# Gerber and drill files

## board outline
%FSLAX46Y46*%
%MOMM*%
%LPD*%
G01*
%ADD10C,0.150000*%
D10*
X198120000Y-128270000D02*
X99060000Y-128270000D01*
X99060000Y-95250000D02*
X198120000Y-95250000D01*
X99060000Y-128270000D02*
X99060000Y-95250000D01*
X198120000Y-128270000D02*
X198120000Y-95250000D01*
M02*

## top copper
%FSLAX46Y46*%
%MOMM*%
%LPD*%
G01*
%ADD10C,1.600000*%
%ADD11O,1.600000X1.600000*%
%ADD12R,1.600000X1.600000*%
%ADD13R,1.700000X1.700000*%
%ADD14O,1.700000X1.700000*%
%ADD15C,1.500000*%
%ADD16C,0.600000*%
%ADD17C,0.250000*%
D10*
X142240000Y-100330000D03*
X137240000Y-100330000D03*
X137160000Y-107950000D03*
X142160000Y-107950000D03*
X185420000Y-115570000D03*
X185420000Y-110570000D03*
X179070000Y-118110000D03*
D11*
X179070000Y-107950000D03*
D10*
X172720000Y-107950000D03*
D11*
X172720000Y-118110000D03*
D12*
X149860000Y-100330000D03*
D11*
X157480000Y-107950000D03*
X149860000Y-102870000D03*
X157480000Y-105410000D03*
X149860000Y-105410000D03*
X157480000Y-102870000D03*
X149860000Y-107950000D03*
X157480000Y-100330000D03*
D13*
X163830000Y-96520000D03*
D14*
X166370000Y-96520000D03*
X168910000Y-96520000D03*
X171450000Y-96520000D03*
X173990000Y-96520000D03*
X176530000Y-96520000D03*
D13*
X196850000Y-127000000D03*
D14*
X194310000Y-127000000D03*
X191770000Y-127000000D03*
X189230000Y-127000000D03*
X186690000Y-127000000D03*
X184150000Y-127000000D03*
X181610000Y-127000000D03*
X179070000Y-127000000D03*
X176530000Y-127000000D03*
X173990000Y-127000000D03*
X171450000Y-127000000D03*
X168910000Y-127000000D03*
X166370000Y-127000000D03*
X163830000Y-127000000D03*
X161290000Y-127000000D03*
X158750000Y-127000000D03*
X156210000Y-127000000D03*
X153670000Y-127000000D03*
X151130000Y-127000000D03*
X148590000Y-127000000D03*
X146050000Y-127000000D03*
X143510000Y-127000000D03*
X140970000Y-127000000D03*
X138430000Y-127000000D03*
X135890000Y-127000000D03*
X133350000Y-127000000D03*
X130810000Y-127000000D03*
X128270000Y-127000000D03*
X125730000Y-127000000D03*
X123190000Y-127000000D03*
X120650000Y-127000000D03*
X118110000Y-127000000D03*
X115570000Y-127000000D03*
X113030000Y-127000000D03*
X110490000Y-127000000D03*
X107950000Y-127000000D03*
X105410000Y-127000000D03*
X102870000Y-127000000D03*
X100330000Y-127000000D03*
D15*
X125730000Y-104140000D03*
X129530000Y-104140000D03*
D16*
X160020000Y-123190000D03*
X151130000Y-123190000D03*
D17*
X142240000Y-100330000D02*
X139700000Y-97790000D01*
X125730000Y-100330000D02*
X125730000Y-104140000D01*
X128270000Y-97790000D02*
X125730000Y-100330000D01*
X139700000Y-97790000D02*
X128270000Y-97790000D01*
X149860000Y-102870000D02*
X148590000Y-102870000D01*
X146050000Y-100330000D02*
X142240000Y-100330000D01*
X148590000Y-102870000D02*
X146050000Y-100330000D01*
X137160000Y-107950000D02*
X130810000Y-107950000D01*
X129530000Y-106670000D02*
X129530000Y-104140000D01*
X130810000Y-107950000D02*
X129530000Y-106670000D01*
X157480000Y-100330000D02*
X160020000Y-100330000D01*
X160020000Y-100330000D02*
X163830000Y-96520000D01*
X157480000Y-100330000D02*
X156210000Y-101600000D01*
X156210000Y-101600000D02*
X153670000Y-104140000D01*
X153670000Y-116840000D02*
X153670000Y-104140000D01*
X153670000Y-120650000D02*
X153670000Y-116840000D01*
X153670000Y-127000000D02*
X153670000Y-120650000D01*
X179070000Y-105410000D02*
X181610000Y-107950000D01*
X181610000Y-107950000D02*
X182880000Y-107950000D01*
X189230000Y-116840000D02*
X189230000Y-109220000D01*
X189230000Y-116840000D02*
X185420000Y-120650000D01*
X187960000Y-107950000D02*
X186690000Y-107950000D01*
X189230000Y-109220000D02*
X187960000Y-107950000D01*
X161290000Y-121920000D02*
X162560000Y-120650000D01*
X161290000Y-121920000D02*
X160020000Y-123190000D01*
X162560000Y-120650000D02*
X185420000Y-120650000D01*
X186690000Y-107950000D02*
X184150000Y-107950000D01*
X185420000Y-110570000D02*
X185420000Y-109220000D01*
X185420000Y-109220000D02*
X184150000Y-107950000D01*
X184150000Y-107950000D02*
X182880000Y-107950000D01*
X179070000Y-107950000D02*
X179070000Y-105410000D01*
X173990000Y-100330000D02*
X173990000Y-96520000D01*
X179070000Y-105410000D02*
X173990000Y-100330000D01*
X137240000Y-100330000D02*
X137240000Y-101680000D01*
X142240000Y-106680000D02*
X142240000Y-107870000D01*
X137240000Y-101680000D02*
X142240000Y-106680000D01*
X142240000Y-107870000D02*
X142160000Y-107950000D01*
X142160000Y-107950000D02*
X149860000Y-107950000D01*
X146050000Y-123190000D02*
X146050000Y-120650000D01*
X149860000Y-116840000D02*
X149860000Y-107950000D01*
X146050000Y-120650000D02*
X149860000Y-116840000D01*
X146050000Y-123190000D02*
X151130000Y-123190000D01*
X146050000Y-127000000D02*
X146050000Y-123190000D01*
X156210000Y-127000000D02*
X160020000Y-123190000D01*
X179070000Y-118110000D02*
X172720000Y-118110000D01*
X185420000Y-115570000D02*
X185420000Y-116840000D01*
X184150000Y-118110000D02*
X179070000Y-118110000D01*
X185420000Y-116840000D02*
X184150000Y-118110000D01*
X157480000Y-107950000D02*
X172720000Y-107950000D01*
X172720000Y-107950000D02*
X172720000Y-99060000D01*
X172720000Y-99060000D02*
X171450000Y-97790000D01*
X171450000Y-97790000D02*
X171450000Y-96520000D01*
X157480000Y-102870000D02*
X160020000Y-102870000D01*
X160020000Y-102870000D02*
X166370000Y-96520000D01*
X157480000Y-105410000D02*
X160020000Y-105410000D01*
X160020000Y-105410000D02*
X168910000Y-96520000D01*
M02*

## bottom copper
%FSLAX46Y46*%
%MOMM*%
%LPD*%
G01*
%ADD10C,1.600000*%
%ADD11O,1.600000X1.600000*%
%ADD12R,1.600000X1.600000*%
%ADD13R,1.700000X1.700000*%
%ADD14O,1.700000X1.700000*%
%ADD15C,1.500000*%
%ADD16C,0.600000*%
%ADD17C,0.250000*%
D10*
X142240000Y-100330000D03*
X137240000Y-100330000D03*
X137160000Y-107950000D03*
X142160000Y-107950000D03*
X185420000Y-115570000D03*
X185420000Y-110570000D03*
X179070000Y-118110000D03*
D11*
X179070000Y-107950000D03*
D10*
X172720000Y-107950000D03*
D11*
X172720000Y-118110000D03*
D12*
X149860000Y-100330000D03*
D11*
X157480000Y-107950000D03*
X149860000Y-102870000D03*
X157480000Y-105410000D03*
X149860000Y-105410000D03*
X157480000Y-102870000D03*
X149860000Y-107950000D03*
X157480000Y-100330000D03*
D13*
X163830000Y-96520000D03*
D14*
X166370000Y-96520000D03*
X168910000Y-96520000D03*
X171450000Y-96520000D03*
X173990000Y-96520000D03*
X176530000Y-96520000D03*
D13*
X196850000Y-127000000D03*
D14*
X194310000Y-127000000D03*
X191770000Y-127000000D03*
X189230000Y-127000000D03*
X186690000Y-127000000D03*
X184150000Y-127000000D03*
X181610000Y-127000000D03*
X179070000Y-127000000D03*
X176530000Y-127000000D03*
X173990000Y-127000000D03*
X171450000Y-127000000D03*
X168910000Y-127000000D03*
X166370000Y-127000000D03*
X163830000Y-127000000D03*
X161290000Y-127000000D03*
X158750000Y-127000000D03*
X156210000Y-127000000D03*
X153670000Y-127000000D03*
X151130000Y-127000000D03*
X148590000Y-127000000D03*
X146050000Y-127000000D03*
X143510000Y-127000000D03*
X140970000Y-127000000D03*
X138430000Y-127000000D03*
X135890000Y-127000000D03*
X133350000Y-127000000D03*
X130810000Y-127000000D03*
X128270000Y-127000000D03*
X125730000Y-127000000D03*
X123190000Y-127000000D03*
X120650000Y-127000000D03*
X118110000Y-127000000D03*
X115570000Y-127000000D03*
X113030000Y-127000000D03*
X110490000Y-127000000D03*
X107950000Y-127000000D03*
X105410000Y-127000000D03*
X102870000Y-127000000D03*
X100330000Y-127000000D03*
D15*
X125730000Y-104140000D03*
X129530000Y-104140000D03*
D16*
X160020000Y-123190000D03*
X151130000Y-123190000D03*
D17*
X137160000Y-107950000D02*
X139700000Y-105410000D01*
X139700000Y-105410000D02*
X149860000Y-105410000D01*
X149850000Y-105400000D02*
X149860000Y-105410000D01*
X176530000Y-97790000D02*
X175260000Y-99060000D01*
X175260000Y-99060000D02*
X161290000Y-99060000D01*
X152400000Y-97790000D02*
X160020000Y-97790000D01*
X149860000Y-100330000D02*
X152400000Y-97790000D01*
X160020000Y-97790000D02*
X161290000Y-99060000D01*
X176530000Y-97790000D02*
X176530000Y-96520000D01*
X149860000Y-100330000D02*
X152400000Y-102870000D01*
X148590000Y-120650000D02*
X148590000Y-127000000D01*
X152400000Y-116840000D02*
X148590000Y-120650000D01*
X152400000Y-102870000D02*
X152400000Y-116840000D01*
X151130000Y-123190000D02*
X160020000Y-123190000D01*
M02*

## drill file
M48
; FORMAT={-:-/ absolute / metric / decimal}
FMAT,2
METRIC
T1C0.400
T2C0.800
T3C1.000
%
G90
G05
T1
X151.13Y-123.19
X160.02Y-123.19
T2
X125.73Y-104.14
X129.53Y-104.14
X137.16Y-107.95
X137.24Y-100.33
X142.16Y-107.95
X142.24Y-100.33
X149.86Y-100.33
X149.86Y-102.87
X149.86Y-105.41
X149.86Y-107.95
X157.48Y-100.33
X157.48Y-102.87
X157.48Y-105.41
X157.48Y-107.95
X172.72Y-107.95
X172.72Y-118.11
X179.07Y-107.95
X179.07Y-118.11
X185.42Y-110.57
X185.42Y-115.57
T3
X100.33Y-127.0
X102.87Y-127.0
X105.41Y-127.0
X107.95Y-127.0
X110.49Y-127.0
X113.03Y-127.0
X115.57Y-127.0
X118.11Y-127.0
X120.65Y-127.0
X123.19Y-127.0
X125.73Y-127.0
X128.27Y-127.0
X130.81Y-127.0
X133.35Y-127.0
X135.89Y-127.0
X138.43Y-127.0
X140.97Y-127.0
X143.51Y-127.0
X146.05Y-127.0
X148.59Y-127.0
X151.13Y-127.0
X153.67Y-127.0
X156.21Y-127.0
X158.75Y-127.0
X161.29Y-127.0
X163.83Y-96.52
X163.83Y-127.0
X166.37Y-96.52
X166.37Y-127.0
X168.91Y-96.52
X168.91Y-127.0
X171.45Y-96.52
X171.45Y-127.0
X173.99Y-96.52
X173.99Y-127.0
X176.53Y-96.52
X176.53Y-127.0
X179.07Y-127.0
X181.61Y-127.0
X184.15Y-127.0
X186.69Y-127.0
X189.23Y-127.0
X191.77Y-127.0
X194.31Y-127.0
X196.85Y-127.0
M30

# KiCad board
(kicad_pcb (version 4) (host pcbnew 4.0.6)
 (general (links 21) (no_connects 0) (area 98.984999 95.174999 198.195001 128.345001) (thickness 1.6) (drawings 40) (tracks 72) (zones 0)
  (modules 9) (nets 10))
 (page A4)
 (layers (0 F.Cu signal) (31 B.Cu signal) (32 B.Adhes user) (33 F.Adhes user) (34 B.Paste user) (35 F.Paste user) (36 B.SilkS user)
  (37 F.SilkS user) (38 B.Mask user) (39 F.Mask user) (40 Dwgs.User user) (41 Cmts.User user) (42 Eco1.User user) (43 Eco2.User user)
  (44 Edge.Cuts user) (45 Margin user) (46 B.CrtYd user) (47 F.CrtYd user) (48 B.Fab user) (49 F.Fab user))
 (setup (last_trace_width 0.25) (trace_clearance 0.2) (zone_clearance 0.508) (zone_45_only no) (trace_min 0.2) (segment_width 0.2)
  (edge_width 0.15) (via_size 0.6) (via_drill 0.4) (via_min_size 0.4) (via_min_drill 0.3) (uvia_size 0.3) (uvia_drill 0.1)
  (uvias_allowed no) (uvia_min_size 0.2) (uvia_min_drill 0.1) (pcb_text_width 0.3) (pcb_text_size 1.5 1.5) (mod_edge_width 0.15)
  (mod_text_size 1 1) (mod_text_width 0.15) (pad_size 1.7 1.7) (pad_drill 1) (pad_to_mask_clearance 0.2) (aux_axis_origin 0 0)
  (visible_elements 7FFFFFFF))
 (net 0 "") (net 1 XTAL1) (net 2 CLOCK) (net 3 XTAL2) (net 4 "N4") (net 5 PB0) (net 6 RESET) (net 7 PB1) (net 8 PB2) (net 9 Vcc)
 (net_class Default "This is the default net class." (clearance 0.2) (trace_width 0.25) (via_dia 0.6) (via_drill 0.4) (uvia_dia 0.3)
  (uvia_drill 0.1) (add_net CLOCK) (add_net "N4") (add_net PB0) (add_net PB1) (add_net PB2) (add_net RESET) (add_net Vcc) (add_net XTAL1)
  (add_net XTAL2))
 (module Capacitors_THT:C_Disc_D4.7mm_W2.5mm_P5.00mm (layer F.Cu) (at 142.24 100.33 180)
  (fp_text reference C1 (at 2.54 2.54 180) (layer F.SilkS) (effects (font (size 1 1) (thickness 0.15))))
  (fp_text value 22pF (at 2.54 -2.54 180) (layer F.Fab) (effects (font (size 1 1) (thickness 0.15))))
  (pad 1 thru_hole circle (at 0 0 180) (size 1.6 1.6) (drill 0.8) (layers *.Cu *.Mask) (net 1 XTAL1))
  (pad 2 thru_hole circle (at 5 0 180) (size 1.6 1.6) (drill 0.8) (layers *.Cu *.Mask) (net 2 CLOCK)))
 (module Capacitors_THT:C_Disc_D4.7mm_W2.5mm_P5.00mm (layer F.Cu) (at 137.16 107.95)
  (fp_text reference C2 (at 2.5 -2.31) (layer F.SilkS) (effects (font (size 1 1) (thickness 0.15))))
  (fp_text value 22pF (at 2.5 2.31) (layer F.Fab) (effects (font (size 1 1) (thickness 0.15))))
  (pad 1 thru_hole circle (at 0 0) (size 1.6 1.6) (drill 0.8) (layers *.Cu *.Mask) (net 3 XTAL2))
  (pad 2 thru_hole circle (at 5 0) (size 1.6 1.6) (drill 0.8) (layers *.Cu *.Mask) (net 2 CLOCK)))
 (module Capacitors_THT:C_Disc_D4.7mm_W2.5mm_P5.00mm (layer F.Cu) (at 185.42 115.57 90)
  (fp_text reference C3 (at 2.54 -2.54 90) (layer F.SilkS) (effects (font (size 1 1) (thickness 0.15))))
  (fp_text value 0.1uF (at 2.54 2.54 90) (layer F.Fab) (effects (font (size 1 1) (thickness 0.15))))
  (pad 1 thru_hole circle (at 0 0 90) (size 1.6 1.6) (drill 0.8) (layers *.Cu *.Mask) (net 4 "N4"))
  (pad 2 thru_hole circle (at 5 0 90) (size 1.6 1.6) (drill 0.8) (layers *.Cu *.Mask) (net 2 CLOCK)))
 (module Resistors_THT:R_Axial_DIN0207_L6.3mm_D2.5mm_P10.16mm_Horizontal (layer F.Cu) (at 179.07 118.11 90)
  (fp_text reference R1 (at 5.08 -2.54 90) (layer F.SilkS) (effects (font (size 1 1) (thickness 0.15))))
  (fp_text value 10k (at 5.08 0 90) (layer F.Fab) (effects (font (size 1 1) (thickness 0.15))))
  (pad 1 thru_hole circle (at 0 0 90) (size 1.6 1.6) (drill 0.8) (layers *.Cu *.Mask) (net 4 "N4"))
  (pad 2 thru_hole oval (at 10.16 0 90) (size 1.6 1.6) (drill 0.8) (layers *.Cu *.Mask) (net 2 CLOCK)))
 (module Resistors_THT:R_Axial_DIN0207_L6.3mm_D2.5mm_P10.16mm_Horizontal (layer F.Cu) (at 172.72 107.95 270)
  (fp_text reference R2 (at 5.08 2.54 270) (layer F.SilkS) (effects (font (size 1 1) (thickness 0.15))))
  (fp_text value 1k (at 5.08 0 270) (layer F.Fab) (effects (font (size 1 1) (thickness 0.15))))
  (pad 1 thru_hole circle (at 0 0 270) (size 1.6 1.6) (drill 0.8) (layers *.Cu *.Mask) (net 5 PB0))
  (pad 2 thru_hole oval (at 10.16 0 270) (size 1.6 1.6) (drill 0.8) (layers *.Cu *.Mask) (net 4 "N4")))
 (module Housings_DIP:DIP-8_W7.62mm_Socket (layer F.Cu) (at 149.86 100.33)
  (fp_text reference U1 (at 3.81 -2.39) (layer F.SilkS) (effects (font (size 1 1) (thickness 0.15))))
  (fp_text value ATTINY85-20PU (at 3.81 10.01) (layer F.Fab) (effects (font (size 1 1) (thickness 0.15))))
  (pad 1 thru_hole rect (at 0 0) (size 1.6 1.6) (drill 0.8) (layers *.Cu *.Mask) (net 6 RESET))
  (pad 5 thru_hole oval (at 7.62 7.62) (size 1.6 1.6) (drill 0.8) (layers *.Cu *.Mask) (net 5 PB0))
  (pad 2 thru_hole oval (at 0 2.54) (size 1.6 1.6) (drill 0.8) (layers *.Cu *.Mask) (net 1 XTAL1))
  (pad 6 thru_hole oval (at 7.62 5.08) (size 1.6 1.6) (drill 0.8) (layers *.Cu *.Mask) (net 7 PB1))
  (pad 3 thru_hole oval (at 0 5.08) (size 1.6 1.6) (drill 0.8) (layers *.Cu *.Mask) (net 3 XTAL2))
  (pad 7 thru_hole oval (at 7.62 2.54) (size 1.6 1.6) (drill 0.8) (layers *.Cu *.Mask) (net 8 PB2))
  (pad 4 thru_hole oval (at 0 7.62) (size 1.6 1.6) (drill 0.8) (layers *.Cu *.Mask) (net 2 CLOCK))
  (pad 8 thru_hole oval (at 7.62 0) (size 1.6 1.6) (drill 0.8) (layers *.Cu *.Mask) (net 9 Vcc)))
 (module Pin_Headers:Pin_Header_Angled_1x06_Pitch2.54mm (layer F.Cu) (at 163.83 96.52 90)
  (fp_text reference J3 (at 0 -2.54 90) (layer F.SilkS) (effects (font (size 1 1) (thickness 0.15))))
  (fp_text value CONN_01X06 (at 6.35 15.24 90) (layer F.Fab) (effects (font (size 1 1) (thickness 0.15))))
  (pad 1 thru_hole rect (at 0 0 90) (size 1.7 1.7) (drill 1) (layers *.Cu *.Mask) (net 9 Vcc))
  (pad 2 thru_hole oval (at 0 2.54 90) (size 1.7 1.7) (drill 1) (layers *.Cu *.Mask) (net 8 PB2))
  (pad 3 thru_hole oval (at 0 5.08 90) (size 1.7 1.7) (drill 1) (layers *.Cu *.Mask) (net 7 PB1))
  (pad 4 thru_hole oval (at 0 7.62 90) (size 1.7 1.7) (drill 1) (layers *.Cu *.Mask) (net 5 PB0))
  (pad 5 thru_hole oval (at 0 10.16 90) (size 1.7 1.7) (drill 1) (layers *.Cu *.Mask) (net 2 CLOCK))
  (pad 6 thru_hole oval (at 0 12.7 90) (size 1.7 1.7) (drill 1) (layers *.Cu *.Mask) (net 6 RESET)))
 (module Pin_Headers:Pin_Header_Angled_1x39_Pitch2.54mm (layer F.Cu) (at 196.85 127 270)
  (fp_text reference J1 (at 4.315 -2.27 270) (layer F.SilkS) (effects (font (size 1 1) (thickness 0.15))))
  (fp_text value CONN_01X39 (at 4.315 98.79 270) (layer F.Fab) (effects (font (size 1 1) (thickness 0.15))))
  (pad 1 thru_hole rect (at 0 0 270) (size 1.7 1.7) (drill 1) (layers *.Cu *.Mask))
  (pad 2 thru_hole oval (at 0 2.54 270) (size 1.7 1.7) (drill 1) (layers *.Cu *.Mask))
  (pad 3 thru_hole oval (at 0 5.08 270) (size 1.7 1.7) (drill 1) (layers *.Cu *.Mask))
  (pad 4 thru_hole oval (at 0 7.62 270) (size 1.7 1.7) (drill 1) (layers *.Cu *.Mask))
  (pad 5 thru_hole oval (at 0 10.16 270) (size 1.7 1.7) (drill 1) (layers *.Cu *.Mask))
  (pad 6 thru_hole oval (at 0 12.7 270) (size 1.7 1.7) (drill 1) (layers *.Cu *.Mask))
  (pad 7 thru_hole oval (at 0 15.24 270) (size 1.7 1.7) (drill 1) (layers *.Cu *.Mask))
  (pad 8 thru_hole oval (at 0 17.78 270) (size 1.7 1.7) (drill 1) (layers *.Cu *.Mask))
  (pad 9 thru_hole oval (at 0 20.32 270) (size 1.7 1.7) (drill 1) (layers *.Cu *.Mask))
  (pad 10 thru_hole oval (at 0 22.86 270) (size 1.7 1.7) (drill 1) (layers *.Cu *.Mask))
  (pad 11 thru_hole oval (at 0 25.4 270) (size 1.7 1.7) (drill 1) (layers *.Cu *.Mask))
  (pad 12 thru_hole oval (at 0 27.94 270) (size 1.7 1.7) (drill 1) (layers *.Cu *.Mask))
  (pad 13 thru_hole oval (at 0 30.48 270) (size 1.7 1.7) (drill 1) (layers *.Cu *.Mask))
  (pad 14 thru_hole oval (at 0 33.02 270) (size 1.7 1.7) (drill 1) (layers *.Cu *.Mask))
  (pad 15 thru_hole oval (at 0 35.56 270) (size 1.7 1.7) (drill 1) (layers *.Cu *.Mask))
  (pad 16 thru_hole oval (at 0 38.1 270) (size 1.7 1.7) (drill 1) (layers *.Cu *.Mask))
  (pad 17 thru_hole oval (at 0 40.64 270) (size 1.7 1.7) (drill 1) (layers *.Cu *.Mask) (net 2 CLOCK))
  (pad 18 thru_hole oval (at 0 43.18 270) (size 1.7 1.7) (drill 1) (layers *.Cu *.Mask) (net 9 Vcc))
  (pad 19 thru_hole oval (at 0 45.72 270) (size 1.7 1.7) (drill 1) (layers *.Cu *.Mask))
  (pad 20 thru_hole oval (at 0 48.26 270) (size 1.7 1.7) (drill 1) (layers *.Cu *.Mask) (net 6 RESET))
  (pad 21 thru_hole oval (at 0 50.8 270) (size 1.7 1.7) (drill 1) (layers *.Cu *.Mask) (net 2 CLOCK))
  (pad 22 thru_hole oval (at 0 53.34 270) (size 1.7 1.7) (drill 1) (layers *.Cu *.Mask))
  (pad 23 thru_hole oval (at 0 55.88 270) (size 1.7 1.7) (drill 1) (layers *.Cu *.Mask))
  (pad 24 thru_hole oval (at 0 58.42 270) (size 1.7 1.7) (drill 1) (layers *.Cu *.Mask))
  (pad 25 thru_hole oval (at 0 60.96 270) (size 1.7 1.7) (drill 1) (layers *.Cu *.Mask))
  (pad 26 thru_hole oval (at 0 63.5 270) (size 1.7 1.7) (drill 1) (layers *.Cu *.Mask))
  (pad 27 thru_hole oval (at 0 66.04 270) (size 1.7 1.7) (drill 1) (layers *.Cu *.Mask))
  (pad 28 thru_hole oval (at 0 68.58 270) (size 1.7 1.7) (drill 1) (layers *.Cu *.Mask))
  (pad 29 thru_hole oval (at 0 71.12 270) (size 1.7 1.7) (drill 1) (layers *.Cu *.Mask))
  (pad 30 thru_hole oval (at 0 73.66 270) (size 1.7 1.7) (drill 1) (layers *.Cu *.Mask))
  (pad 31 thru_hole oval (at 0 76.2 270) (size 1.7 1.7) (drill 1) (layers *.Cu *.Mask))
  (pad 32 thru_hole oval (at 0 78.74 270) (size 1.7 1.7) (drill 1) (layers *.Cu *.Mask))
  (pad 33 thru_hole oval (at 0 81.28 270) (size 1.7 1.7) (drill 1) (layers *.Cu *.Mask))
  (pad 34 thru_hole oval (at 0 83.82 270) (size 1.7 1.7) (drill 1) (layers *.Cu *.Mask))
  (pad 35 thru_hole oval (at 0 86.36 270) (size 1.7 1.7) (drill 1) (layers *.Cu *.Mask))
  (pad 36 thru_hole oval (at 0 88.9 270) (size 1.7 1.7) (drill 1) (layers *.Cu *.Mask))
  (pad 37 thru_hole oval (at 0 91.44 270) (size 1.7 1.7) (drill 1) (layers *.Cu *.Mask))
  (pad 38 thru_hole oval (at 0 93.98 270) (size 1.7 1.7) (drill 1) (layers *.Cu *.Mask))
  (pad 39 thru_hole oval (at 0 96.52 270) (size 1.7 1.7) (drill 1) (layers *.Cu *.Mask)))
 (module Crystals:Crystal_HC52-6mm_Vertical (layer F.Cu) (at 125.73 104.14)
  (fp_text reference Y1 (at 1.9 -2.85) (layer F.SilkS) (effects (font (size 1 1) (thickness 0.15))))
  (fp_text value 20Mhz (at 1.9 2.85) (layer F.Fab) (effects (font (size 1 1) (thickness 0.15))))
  (pad 1 thru_hole circle (at 0 0) (size 1.5 1.5) (drill 0.8) (layers *.Cu *.Mask) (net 1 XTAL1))
  (pad 2 thru_hole circle (at 3.8 0) (size 1.5 1.5) (drill 0.8) (layers *.Cu *.Mask) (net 3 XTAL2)))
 (gr_line (start 198.12 128.27) (end 99.06 128.27) (angle 90) (layer Edge.Cuts) (width 0.15))
 (gr_line (start 99.06 95.25) (end 198.12 95.25) (angle 90) (layer Edge.Cuts) (width 0.15))
 (gr_line (start 99.06 128.27) (end 99.06 95.25) (angle 90) (layer Edge.Cuts) (width 0.15))
 (gr_line (start 198.12 128.27) (end 198.12 95.25) (angle 90) (layer Edge.Cuts) (width 0.15))
 (segment (start 142.24 100.33) (end 139.7 97.79) (width 0.25) (layer F.Cu) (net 1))
 (segment (start 125.73 100.33) (end 125.73 104.14) (width 0.25) (layer F.Cu) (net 1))
 (segment (start 128.27 97.79) (end 125.73 100.33) (width 0.25) (layer F.Cu) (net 1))
 (segment (start 139.7 97.79) (end 128.27 97.79) (width 0.25) (layer F.Cu) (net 1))
 (segment (start 149.86 102.87) (end 148.59 102.87) (width 0.25) (layer F.Cu) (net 1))
 (segment (start 146.05 100.33) (end 142.24 100.33) (width 0.25) (layer F.Cu) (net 1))
 (segment (start 148.59 102.87) (end 146.05 100.33) (width 0.25) (layer F.Cu) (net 1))
 (segment (start 137.16 107.95) (end 139.7 105.41) (width 0.25) (layer B.Cu) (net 3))
 (segment (start 139.7 105.41) (end 149.86 105.41) (width 0.25) (layer B.Cu) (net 3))
 (segment (start 137.16 107.95) (end 130.81 107.95) (width 0.25) (layer F.Cu) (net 3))
 (segment (start 129.53 106.67) (end 129.53 104.14) (width 0.25) (layer F.Cu) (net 3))
 (segment (start 130.81 107.95) (end 129.53 106.67) (width 0.25) (layer F.Cu) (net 3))
 (segment (start 149.85 105.4) (end 149.86 105.41) (width 0.25) (layer B.Cu) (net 3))
 (segment (start 157.48 100.33) (end 160.02 100.33) (width 0.25) (layer F.Cu) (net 9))
 (segment (start 160.02 100.33) (end 163.83 96.52) (width 0.25) (layer F.Cu) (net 9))
 (segment (start 157.48 100.33) (end 156.21 101.6) (width 0.25) (layer F.Cu) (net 9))
 (segment (start 156.21 101.6) (end 153.67 104.14) (width 0.25) (layer F.Cu) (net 9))
 (segment (start 153.67 116.84) (end 153.67 104.14) (width 0.25) (layer F.Cu) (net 9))
 (segment (start 153.67 120.65) (end 153.67 116.84) (width 0.25) (layer F.Cu) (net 9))
 (segment (start 153.67 127) (end 153.67 120.65) (width 0.25) (layer F.Cu) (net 9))
 (segment (start 176.53 97.79) (end 175.26 99.06) (width 0.25) (layer B.Cu) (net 6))
 (segment (start 175.26 99.06) (end 161.29 99.06) (width 0.25) (layer B.Cu) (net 6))
 (segment (start 152.4 97.79) (end 160.02 97.79) (width 0.25) (layer B.Cu) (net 6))
 (segment (start 149.86 100.33) (end 152.4 97.79) (width 0.25) (layer B.Cu) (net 6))
 (segment (start 160.02 97.79) (end 161.29 99.06) (width 0.25) (layer B.Cu) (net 6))
 (segment (start 176.53 97.79) (end 176.53 96.52) (width 0.25) (layer B.Cu) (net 6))
 (segment (start 149.86 100.33) (end 152.4 102.87) (width 0.25) (layer B.Cu) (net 6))
 (segment (start 148.59 120.65) (end 148.59 127) (width 0.25) (layer B.Cu) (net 6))
 (segment (start 152.4 116.84) (end 148.59 120.65) (width 0.25) (layer B.Cu) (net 6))
 (segment (start 152.4 102.87) (end 152.4 116.84) (width 0.25) (layer B.Cu) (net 6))
 (segment (start 179.07 105.41) (end 181.61 107.95) (width 0.25) (layer F.Cu) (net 2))
 (segment (start 181.61 107.95) (end 182.88 107.95) (width 0.25) (layer F.Cu) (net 2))
 (segment (start 189.23 116.84) (end 189.23 109.22) (width 0.25) (layer F.Cu) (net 2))
 (segment (start 189.23 116.84) (end 185.42 120.65) (width 0.25) (layer F.Cu) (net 2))
 (segment (start 187.96 107.95) (end 186.69 107.95) (width 0.25) (layer F.Cu) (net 2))
 (segment (start 189.23 109.22) (end 187.96 107.95) (width 0.25) (layer F.Cu) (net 2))
 (segment (start 161.29 121.92) (end 162.56 120.65) (width 0.25) (layer F.Cu) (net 2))
 (segment (start 161.29 121.92) (end 160.02 123.19) (width 0.25) (layer F.Cu) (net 2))
 (segment (start 162.56 120.65) (end 185.42 120.65) (width 0.25) (layer F.Cu) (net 2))
 (segment (start 186.69 107.95) (end 184.15 107.95) (width 0.25) (layer F.Cu) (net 2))
 (segment (start 185.42 110.57) (end 185.42 109.22) (width 0.25) (layer F.Cu) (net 2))
 (segment (start 185.42 109.22) (end 184.15 107.95) (width 0.25) (layer F.Cu) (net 2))
 (segment (start 184.15 107.95) (end 182.88 107.95) (width 0.25) (layer F.Cu) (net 2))
 (segment (start 179.07 107.95) (end 179.07 105.41) (width 0.25) (layer F.Cu) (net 2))
 (segment (start 173.99 100.33) (end 173.99 96.52) (width 0.25) (layer F.Cu) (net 2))
 (segment (start 179.07 105.41) (end 173.99 100.33) (width 0.25) (layer F.Cu) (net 2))
 (segment (start 137.24 100.33) (end 137.24 101.68) (width 0.25) (layer F.Cu) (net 2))
 (segment (start 142.24 106.68) (end 142.24 107.87) (width 0.25) (layer F.Cu) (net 2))
 (segment (start 137.24 101.68) (end 142.24 106.68) (width 0.25) (layer F.Cu) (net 2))
 (segment (start 142.24 107.87) (end 142.16 107.95) (width 0.25) (layer F.Cu) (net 2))
 (segment (start 142.16 107.95) (end 149.86 107.95) (width 0.25) (layer F.Cu) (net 2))
 (segment (start 146.05 123.19) (end 146.05 120.65) (width 0.25) (layer F.Cu) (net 2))
 (segment (start 149.86 116.84) (end 149.86 107.95) (width 0.25) (layer F.Cu) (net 2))
 (segment (start 146.05 120.65) (end 149.86 116.84) (width 0.25) (layer F.Cu) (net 2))
 (segment (start 146.05 123.19) (end 151.13 123.19) (width 0.25) (layer F.Cu) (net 2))
 (via (at 160.02 123.19) (size 0.6) (drill 0.4) (layers F.Cu B.Cu) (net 2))
 (segment (start 151.13 123.19) (end 160.02 123.19) (width 0.25) (layer B.Cu) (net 2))
 (via (at 151.13 123.19) (size 0.6) (drill 0.4) (layers F.Cu B.Cu) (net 2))
 (segment (start 146.05 127) (end 146.05 123.19) (width 0.25) (layer F.Cu) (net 2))
 (segment (start 156.21 127) (end 160.02 123.19) (width 0.25) (layer F.Cu) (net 2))
 (segment (start 179.07 118.11) (end 172.72 118.11) (width 0.25) (layer F.Cu) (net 4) (status C00000))
 (segment (start 185.42 115.57) (end 185.42 116.84) (width 0.25) (layer F.Cu) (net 4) (status 400000))
 (segment (start 184.15 118.11) (end 179.07 118.11) (width 0.25) (layer F.Cu) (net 4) (status 800000))
 (segment (start 185.42 116.84) (end 184.15 118.11) (width 0.25) (layer F.Cu) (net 4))
 (segment (start 157.48 107.95) (end 172.72 107.95) (width 0.25) (layer F.Cu) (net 5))
 (segment (start 172.72 107.95) (end 172.72 99.06) (width 0.25) (layer F.Cu) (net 5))
 (segment (start 172.72 99.06) (end 171.45 97.79) (width 0.25) (layer F.Cu) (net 5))
 (segment (start 171.45 97.79) (end 171.45 96.52) (width 0.25) (layer F.Cu) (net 5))
 (segment (start 157.48 102.87) (end 160.02 102.87) (width 0.25) (layer F.Cu) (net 8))
 (segment (start 160.02 102.87) (end 166.37 96.52) (width 0.25) (layer F.Cu) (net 8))
 (segment (start 157.48 105.41) (end 160.02 105.41) (width 0.25) (layer F.Cu) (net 7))
 (segment (start 160.02 105.41) (end 168.91 96.52) (width 0.25) (layer F.Cu) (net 7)))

